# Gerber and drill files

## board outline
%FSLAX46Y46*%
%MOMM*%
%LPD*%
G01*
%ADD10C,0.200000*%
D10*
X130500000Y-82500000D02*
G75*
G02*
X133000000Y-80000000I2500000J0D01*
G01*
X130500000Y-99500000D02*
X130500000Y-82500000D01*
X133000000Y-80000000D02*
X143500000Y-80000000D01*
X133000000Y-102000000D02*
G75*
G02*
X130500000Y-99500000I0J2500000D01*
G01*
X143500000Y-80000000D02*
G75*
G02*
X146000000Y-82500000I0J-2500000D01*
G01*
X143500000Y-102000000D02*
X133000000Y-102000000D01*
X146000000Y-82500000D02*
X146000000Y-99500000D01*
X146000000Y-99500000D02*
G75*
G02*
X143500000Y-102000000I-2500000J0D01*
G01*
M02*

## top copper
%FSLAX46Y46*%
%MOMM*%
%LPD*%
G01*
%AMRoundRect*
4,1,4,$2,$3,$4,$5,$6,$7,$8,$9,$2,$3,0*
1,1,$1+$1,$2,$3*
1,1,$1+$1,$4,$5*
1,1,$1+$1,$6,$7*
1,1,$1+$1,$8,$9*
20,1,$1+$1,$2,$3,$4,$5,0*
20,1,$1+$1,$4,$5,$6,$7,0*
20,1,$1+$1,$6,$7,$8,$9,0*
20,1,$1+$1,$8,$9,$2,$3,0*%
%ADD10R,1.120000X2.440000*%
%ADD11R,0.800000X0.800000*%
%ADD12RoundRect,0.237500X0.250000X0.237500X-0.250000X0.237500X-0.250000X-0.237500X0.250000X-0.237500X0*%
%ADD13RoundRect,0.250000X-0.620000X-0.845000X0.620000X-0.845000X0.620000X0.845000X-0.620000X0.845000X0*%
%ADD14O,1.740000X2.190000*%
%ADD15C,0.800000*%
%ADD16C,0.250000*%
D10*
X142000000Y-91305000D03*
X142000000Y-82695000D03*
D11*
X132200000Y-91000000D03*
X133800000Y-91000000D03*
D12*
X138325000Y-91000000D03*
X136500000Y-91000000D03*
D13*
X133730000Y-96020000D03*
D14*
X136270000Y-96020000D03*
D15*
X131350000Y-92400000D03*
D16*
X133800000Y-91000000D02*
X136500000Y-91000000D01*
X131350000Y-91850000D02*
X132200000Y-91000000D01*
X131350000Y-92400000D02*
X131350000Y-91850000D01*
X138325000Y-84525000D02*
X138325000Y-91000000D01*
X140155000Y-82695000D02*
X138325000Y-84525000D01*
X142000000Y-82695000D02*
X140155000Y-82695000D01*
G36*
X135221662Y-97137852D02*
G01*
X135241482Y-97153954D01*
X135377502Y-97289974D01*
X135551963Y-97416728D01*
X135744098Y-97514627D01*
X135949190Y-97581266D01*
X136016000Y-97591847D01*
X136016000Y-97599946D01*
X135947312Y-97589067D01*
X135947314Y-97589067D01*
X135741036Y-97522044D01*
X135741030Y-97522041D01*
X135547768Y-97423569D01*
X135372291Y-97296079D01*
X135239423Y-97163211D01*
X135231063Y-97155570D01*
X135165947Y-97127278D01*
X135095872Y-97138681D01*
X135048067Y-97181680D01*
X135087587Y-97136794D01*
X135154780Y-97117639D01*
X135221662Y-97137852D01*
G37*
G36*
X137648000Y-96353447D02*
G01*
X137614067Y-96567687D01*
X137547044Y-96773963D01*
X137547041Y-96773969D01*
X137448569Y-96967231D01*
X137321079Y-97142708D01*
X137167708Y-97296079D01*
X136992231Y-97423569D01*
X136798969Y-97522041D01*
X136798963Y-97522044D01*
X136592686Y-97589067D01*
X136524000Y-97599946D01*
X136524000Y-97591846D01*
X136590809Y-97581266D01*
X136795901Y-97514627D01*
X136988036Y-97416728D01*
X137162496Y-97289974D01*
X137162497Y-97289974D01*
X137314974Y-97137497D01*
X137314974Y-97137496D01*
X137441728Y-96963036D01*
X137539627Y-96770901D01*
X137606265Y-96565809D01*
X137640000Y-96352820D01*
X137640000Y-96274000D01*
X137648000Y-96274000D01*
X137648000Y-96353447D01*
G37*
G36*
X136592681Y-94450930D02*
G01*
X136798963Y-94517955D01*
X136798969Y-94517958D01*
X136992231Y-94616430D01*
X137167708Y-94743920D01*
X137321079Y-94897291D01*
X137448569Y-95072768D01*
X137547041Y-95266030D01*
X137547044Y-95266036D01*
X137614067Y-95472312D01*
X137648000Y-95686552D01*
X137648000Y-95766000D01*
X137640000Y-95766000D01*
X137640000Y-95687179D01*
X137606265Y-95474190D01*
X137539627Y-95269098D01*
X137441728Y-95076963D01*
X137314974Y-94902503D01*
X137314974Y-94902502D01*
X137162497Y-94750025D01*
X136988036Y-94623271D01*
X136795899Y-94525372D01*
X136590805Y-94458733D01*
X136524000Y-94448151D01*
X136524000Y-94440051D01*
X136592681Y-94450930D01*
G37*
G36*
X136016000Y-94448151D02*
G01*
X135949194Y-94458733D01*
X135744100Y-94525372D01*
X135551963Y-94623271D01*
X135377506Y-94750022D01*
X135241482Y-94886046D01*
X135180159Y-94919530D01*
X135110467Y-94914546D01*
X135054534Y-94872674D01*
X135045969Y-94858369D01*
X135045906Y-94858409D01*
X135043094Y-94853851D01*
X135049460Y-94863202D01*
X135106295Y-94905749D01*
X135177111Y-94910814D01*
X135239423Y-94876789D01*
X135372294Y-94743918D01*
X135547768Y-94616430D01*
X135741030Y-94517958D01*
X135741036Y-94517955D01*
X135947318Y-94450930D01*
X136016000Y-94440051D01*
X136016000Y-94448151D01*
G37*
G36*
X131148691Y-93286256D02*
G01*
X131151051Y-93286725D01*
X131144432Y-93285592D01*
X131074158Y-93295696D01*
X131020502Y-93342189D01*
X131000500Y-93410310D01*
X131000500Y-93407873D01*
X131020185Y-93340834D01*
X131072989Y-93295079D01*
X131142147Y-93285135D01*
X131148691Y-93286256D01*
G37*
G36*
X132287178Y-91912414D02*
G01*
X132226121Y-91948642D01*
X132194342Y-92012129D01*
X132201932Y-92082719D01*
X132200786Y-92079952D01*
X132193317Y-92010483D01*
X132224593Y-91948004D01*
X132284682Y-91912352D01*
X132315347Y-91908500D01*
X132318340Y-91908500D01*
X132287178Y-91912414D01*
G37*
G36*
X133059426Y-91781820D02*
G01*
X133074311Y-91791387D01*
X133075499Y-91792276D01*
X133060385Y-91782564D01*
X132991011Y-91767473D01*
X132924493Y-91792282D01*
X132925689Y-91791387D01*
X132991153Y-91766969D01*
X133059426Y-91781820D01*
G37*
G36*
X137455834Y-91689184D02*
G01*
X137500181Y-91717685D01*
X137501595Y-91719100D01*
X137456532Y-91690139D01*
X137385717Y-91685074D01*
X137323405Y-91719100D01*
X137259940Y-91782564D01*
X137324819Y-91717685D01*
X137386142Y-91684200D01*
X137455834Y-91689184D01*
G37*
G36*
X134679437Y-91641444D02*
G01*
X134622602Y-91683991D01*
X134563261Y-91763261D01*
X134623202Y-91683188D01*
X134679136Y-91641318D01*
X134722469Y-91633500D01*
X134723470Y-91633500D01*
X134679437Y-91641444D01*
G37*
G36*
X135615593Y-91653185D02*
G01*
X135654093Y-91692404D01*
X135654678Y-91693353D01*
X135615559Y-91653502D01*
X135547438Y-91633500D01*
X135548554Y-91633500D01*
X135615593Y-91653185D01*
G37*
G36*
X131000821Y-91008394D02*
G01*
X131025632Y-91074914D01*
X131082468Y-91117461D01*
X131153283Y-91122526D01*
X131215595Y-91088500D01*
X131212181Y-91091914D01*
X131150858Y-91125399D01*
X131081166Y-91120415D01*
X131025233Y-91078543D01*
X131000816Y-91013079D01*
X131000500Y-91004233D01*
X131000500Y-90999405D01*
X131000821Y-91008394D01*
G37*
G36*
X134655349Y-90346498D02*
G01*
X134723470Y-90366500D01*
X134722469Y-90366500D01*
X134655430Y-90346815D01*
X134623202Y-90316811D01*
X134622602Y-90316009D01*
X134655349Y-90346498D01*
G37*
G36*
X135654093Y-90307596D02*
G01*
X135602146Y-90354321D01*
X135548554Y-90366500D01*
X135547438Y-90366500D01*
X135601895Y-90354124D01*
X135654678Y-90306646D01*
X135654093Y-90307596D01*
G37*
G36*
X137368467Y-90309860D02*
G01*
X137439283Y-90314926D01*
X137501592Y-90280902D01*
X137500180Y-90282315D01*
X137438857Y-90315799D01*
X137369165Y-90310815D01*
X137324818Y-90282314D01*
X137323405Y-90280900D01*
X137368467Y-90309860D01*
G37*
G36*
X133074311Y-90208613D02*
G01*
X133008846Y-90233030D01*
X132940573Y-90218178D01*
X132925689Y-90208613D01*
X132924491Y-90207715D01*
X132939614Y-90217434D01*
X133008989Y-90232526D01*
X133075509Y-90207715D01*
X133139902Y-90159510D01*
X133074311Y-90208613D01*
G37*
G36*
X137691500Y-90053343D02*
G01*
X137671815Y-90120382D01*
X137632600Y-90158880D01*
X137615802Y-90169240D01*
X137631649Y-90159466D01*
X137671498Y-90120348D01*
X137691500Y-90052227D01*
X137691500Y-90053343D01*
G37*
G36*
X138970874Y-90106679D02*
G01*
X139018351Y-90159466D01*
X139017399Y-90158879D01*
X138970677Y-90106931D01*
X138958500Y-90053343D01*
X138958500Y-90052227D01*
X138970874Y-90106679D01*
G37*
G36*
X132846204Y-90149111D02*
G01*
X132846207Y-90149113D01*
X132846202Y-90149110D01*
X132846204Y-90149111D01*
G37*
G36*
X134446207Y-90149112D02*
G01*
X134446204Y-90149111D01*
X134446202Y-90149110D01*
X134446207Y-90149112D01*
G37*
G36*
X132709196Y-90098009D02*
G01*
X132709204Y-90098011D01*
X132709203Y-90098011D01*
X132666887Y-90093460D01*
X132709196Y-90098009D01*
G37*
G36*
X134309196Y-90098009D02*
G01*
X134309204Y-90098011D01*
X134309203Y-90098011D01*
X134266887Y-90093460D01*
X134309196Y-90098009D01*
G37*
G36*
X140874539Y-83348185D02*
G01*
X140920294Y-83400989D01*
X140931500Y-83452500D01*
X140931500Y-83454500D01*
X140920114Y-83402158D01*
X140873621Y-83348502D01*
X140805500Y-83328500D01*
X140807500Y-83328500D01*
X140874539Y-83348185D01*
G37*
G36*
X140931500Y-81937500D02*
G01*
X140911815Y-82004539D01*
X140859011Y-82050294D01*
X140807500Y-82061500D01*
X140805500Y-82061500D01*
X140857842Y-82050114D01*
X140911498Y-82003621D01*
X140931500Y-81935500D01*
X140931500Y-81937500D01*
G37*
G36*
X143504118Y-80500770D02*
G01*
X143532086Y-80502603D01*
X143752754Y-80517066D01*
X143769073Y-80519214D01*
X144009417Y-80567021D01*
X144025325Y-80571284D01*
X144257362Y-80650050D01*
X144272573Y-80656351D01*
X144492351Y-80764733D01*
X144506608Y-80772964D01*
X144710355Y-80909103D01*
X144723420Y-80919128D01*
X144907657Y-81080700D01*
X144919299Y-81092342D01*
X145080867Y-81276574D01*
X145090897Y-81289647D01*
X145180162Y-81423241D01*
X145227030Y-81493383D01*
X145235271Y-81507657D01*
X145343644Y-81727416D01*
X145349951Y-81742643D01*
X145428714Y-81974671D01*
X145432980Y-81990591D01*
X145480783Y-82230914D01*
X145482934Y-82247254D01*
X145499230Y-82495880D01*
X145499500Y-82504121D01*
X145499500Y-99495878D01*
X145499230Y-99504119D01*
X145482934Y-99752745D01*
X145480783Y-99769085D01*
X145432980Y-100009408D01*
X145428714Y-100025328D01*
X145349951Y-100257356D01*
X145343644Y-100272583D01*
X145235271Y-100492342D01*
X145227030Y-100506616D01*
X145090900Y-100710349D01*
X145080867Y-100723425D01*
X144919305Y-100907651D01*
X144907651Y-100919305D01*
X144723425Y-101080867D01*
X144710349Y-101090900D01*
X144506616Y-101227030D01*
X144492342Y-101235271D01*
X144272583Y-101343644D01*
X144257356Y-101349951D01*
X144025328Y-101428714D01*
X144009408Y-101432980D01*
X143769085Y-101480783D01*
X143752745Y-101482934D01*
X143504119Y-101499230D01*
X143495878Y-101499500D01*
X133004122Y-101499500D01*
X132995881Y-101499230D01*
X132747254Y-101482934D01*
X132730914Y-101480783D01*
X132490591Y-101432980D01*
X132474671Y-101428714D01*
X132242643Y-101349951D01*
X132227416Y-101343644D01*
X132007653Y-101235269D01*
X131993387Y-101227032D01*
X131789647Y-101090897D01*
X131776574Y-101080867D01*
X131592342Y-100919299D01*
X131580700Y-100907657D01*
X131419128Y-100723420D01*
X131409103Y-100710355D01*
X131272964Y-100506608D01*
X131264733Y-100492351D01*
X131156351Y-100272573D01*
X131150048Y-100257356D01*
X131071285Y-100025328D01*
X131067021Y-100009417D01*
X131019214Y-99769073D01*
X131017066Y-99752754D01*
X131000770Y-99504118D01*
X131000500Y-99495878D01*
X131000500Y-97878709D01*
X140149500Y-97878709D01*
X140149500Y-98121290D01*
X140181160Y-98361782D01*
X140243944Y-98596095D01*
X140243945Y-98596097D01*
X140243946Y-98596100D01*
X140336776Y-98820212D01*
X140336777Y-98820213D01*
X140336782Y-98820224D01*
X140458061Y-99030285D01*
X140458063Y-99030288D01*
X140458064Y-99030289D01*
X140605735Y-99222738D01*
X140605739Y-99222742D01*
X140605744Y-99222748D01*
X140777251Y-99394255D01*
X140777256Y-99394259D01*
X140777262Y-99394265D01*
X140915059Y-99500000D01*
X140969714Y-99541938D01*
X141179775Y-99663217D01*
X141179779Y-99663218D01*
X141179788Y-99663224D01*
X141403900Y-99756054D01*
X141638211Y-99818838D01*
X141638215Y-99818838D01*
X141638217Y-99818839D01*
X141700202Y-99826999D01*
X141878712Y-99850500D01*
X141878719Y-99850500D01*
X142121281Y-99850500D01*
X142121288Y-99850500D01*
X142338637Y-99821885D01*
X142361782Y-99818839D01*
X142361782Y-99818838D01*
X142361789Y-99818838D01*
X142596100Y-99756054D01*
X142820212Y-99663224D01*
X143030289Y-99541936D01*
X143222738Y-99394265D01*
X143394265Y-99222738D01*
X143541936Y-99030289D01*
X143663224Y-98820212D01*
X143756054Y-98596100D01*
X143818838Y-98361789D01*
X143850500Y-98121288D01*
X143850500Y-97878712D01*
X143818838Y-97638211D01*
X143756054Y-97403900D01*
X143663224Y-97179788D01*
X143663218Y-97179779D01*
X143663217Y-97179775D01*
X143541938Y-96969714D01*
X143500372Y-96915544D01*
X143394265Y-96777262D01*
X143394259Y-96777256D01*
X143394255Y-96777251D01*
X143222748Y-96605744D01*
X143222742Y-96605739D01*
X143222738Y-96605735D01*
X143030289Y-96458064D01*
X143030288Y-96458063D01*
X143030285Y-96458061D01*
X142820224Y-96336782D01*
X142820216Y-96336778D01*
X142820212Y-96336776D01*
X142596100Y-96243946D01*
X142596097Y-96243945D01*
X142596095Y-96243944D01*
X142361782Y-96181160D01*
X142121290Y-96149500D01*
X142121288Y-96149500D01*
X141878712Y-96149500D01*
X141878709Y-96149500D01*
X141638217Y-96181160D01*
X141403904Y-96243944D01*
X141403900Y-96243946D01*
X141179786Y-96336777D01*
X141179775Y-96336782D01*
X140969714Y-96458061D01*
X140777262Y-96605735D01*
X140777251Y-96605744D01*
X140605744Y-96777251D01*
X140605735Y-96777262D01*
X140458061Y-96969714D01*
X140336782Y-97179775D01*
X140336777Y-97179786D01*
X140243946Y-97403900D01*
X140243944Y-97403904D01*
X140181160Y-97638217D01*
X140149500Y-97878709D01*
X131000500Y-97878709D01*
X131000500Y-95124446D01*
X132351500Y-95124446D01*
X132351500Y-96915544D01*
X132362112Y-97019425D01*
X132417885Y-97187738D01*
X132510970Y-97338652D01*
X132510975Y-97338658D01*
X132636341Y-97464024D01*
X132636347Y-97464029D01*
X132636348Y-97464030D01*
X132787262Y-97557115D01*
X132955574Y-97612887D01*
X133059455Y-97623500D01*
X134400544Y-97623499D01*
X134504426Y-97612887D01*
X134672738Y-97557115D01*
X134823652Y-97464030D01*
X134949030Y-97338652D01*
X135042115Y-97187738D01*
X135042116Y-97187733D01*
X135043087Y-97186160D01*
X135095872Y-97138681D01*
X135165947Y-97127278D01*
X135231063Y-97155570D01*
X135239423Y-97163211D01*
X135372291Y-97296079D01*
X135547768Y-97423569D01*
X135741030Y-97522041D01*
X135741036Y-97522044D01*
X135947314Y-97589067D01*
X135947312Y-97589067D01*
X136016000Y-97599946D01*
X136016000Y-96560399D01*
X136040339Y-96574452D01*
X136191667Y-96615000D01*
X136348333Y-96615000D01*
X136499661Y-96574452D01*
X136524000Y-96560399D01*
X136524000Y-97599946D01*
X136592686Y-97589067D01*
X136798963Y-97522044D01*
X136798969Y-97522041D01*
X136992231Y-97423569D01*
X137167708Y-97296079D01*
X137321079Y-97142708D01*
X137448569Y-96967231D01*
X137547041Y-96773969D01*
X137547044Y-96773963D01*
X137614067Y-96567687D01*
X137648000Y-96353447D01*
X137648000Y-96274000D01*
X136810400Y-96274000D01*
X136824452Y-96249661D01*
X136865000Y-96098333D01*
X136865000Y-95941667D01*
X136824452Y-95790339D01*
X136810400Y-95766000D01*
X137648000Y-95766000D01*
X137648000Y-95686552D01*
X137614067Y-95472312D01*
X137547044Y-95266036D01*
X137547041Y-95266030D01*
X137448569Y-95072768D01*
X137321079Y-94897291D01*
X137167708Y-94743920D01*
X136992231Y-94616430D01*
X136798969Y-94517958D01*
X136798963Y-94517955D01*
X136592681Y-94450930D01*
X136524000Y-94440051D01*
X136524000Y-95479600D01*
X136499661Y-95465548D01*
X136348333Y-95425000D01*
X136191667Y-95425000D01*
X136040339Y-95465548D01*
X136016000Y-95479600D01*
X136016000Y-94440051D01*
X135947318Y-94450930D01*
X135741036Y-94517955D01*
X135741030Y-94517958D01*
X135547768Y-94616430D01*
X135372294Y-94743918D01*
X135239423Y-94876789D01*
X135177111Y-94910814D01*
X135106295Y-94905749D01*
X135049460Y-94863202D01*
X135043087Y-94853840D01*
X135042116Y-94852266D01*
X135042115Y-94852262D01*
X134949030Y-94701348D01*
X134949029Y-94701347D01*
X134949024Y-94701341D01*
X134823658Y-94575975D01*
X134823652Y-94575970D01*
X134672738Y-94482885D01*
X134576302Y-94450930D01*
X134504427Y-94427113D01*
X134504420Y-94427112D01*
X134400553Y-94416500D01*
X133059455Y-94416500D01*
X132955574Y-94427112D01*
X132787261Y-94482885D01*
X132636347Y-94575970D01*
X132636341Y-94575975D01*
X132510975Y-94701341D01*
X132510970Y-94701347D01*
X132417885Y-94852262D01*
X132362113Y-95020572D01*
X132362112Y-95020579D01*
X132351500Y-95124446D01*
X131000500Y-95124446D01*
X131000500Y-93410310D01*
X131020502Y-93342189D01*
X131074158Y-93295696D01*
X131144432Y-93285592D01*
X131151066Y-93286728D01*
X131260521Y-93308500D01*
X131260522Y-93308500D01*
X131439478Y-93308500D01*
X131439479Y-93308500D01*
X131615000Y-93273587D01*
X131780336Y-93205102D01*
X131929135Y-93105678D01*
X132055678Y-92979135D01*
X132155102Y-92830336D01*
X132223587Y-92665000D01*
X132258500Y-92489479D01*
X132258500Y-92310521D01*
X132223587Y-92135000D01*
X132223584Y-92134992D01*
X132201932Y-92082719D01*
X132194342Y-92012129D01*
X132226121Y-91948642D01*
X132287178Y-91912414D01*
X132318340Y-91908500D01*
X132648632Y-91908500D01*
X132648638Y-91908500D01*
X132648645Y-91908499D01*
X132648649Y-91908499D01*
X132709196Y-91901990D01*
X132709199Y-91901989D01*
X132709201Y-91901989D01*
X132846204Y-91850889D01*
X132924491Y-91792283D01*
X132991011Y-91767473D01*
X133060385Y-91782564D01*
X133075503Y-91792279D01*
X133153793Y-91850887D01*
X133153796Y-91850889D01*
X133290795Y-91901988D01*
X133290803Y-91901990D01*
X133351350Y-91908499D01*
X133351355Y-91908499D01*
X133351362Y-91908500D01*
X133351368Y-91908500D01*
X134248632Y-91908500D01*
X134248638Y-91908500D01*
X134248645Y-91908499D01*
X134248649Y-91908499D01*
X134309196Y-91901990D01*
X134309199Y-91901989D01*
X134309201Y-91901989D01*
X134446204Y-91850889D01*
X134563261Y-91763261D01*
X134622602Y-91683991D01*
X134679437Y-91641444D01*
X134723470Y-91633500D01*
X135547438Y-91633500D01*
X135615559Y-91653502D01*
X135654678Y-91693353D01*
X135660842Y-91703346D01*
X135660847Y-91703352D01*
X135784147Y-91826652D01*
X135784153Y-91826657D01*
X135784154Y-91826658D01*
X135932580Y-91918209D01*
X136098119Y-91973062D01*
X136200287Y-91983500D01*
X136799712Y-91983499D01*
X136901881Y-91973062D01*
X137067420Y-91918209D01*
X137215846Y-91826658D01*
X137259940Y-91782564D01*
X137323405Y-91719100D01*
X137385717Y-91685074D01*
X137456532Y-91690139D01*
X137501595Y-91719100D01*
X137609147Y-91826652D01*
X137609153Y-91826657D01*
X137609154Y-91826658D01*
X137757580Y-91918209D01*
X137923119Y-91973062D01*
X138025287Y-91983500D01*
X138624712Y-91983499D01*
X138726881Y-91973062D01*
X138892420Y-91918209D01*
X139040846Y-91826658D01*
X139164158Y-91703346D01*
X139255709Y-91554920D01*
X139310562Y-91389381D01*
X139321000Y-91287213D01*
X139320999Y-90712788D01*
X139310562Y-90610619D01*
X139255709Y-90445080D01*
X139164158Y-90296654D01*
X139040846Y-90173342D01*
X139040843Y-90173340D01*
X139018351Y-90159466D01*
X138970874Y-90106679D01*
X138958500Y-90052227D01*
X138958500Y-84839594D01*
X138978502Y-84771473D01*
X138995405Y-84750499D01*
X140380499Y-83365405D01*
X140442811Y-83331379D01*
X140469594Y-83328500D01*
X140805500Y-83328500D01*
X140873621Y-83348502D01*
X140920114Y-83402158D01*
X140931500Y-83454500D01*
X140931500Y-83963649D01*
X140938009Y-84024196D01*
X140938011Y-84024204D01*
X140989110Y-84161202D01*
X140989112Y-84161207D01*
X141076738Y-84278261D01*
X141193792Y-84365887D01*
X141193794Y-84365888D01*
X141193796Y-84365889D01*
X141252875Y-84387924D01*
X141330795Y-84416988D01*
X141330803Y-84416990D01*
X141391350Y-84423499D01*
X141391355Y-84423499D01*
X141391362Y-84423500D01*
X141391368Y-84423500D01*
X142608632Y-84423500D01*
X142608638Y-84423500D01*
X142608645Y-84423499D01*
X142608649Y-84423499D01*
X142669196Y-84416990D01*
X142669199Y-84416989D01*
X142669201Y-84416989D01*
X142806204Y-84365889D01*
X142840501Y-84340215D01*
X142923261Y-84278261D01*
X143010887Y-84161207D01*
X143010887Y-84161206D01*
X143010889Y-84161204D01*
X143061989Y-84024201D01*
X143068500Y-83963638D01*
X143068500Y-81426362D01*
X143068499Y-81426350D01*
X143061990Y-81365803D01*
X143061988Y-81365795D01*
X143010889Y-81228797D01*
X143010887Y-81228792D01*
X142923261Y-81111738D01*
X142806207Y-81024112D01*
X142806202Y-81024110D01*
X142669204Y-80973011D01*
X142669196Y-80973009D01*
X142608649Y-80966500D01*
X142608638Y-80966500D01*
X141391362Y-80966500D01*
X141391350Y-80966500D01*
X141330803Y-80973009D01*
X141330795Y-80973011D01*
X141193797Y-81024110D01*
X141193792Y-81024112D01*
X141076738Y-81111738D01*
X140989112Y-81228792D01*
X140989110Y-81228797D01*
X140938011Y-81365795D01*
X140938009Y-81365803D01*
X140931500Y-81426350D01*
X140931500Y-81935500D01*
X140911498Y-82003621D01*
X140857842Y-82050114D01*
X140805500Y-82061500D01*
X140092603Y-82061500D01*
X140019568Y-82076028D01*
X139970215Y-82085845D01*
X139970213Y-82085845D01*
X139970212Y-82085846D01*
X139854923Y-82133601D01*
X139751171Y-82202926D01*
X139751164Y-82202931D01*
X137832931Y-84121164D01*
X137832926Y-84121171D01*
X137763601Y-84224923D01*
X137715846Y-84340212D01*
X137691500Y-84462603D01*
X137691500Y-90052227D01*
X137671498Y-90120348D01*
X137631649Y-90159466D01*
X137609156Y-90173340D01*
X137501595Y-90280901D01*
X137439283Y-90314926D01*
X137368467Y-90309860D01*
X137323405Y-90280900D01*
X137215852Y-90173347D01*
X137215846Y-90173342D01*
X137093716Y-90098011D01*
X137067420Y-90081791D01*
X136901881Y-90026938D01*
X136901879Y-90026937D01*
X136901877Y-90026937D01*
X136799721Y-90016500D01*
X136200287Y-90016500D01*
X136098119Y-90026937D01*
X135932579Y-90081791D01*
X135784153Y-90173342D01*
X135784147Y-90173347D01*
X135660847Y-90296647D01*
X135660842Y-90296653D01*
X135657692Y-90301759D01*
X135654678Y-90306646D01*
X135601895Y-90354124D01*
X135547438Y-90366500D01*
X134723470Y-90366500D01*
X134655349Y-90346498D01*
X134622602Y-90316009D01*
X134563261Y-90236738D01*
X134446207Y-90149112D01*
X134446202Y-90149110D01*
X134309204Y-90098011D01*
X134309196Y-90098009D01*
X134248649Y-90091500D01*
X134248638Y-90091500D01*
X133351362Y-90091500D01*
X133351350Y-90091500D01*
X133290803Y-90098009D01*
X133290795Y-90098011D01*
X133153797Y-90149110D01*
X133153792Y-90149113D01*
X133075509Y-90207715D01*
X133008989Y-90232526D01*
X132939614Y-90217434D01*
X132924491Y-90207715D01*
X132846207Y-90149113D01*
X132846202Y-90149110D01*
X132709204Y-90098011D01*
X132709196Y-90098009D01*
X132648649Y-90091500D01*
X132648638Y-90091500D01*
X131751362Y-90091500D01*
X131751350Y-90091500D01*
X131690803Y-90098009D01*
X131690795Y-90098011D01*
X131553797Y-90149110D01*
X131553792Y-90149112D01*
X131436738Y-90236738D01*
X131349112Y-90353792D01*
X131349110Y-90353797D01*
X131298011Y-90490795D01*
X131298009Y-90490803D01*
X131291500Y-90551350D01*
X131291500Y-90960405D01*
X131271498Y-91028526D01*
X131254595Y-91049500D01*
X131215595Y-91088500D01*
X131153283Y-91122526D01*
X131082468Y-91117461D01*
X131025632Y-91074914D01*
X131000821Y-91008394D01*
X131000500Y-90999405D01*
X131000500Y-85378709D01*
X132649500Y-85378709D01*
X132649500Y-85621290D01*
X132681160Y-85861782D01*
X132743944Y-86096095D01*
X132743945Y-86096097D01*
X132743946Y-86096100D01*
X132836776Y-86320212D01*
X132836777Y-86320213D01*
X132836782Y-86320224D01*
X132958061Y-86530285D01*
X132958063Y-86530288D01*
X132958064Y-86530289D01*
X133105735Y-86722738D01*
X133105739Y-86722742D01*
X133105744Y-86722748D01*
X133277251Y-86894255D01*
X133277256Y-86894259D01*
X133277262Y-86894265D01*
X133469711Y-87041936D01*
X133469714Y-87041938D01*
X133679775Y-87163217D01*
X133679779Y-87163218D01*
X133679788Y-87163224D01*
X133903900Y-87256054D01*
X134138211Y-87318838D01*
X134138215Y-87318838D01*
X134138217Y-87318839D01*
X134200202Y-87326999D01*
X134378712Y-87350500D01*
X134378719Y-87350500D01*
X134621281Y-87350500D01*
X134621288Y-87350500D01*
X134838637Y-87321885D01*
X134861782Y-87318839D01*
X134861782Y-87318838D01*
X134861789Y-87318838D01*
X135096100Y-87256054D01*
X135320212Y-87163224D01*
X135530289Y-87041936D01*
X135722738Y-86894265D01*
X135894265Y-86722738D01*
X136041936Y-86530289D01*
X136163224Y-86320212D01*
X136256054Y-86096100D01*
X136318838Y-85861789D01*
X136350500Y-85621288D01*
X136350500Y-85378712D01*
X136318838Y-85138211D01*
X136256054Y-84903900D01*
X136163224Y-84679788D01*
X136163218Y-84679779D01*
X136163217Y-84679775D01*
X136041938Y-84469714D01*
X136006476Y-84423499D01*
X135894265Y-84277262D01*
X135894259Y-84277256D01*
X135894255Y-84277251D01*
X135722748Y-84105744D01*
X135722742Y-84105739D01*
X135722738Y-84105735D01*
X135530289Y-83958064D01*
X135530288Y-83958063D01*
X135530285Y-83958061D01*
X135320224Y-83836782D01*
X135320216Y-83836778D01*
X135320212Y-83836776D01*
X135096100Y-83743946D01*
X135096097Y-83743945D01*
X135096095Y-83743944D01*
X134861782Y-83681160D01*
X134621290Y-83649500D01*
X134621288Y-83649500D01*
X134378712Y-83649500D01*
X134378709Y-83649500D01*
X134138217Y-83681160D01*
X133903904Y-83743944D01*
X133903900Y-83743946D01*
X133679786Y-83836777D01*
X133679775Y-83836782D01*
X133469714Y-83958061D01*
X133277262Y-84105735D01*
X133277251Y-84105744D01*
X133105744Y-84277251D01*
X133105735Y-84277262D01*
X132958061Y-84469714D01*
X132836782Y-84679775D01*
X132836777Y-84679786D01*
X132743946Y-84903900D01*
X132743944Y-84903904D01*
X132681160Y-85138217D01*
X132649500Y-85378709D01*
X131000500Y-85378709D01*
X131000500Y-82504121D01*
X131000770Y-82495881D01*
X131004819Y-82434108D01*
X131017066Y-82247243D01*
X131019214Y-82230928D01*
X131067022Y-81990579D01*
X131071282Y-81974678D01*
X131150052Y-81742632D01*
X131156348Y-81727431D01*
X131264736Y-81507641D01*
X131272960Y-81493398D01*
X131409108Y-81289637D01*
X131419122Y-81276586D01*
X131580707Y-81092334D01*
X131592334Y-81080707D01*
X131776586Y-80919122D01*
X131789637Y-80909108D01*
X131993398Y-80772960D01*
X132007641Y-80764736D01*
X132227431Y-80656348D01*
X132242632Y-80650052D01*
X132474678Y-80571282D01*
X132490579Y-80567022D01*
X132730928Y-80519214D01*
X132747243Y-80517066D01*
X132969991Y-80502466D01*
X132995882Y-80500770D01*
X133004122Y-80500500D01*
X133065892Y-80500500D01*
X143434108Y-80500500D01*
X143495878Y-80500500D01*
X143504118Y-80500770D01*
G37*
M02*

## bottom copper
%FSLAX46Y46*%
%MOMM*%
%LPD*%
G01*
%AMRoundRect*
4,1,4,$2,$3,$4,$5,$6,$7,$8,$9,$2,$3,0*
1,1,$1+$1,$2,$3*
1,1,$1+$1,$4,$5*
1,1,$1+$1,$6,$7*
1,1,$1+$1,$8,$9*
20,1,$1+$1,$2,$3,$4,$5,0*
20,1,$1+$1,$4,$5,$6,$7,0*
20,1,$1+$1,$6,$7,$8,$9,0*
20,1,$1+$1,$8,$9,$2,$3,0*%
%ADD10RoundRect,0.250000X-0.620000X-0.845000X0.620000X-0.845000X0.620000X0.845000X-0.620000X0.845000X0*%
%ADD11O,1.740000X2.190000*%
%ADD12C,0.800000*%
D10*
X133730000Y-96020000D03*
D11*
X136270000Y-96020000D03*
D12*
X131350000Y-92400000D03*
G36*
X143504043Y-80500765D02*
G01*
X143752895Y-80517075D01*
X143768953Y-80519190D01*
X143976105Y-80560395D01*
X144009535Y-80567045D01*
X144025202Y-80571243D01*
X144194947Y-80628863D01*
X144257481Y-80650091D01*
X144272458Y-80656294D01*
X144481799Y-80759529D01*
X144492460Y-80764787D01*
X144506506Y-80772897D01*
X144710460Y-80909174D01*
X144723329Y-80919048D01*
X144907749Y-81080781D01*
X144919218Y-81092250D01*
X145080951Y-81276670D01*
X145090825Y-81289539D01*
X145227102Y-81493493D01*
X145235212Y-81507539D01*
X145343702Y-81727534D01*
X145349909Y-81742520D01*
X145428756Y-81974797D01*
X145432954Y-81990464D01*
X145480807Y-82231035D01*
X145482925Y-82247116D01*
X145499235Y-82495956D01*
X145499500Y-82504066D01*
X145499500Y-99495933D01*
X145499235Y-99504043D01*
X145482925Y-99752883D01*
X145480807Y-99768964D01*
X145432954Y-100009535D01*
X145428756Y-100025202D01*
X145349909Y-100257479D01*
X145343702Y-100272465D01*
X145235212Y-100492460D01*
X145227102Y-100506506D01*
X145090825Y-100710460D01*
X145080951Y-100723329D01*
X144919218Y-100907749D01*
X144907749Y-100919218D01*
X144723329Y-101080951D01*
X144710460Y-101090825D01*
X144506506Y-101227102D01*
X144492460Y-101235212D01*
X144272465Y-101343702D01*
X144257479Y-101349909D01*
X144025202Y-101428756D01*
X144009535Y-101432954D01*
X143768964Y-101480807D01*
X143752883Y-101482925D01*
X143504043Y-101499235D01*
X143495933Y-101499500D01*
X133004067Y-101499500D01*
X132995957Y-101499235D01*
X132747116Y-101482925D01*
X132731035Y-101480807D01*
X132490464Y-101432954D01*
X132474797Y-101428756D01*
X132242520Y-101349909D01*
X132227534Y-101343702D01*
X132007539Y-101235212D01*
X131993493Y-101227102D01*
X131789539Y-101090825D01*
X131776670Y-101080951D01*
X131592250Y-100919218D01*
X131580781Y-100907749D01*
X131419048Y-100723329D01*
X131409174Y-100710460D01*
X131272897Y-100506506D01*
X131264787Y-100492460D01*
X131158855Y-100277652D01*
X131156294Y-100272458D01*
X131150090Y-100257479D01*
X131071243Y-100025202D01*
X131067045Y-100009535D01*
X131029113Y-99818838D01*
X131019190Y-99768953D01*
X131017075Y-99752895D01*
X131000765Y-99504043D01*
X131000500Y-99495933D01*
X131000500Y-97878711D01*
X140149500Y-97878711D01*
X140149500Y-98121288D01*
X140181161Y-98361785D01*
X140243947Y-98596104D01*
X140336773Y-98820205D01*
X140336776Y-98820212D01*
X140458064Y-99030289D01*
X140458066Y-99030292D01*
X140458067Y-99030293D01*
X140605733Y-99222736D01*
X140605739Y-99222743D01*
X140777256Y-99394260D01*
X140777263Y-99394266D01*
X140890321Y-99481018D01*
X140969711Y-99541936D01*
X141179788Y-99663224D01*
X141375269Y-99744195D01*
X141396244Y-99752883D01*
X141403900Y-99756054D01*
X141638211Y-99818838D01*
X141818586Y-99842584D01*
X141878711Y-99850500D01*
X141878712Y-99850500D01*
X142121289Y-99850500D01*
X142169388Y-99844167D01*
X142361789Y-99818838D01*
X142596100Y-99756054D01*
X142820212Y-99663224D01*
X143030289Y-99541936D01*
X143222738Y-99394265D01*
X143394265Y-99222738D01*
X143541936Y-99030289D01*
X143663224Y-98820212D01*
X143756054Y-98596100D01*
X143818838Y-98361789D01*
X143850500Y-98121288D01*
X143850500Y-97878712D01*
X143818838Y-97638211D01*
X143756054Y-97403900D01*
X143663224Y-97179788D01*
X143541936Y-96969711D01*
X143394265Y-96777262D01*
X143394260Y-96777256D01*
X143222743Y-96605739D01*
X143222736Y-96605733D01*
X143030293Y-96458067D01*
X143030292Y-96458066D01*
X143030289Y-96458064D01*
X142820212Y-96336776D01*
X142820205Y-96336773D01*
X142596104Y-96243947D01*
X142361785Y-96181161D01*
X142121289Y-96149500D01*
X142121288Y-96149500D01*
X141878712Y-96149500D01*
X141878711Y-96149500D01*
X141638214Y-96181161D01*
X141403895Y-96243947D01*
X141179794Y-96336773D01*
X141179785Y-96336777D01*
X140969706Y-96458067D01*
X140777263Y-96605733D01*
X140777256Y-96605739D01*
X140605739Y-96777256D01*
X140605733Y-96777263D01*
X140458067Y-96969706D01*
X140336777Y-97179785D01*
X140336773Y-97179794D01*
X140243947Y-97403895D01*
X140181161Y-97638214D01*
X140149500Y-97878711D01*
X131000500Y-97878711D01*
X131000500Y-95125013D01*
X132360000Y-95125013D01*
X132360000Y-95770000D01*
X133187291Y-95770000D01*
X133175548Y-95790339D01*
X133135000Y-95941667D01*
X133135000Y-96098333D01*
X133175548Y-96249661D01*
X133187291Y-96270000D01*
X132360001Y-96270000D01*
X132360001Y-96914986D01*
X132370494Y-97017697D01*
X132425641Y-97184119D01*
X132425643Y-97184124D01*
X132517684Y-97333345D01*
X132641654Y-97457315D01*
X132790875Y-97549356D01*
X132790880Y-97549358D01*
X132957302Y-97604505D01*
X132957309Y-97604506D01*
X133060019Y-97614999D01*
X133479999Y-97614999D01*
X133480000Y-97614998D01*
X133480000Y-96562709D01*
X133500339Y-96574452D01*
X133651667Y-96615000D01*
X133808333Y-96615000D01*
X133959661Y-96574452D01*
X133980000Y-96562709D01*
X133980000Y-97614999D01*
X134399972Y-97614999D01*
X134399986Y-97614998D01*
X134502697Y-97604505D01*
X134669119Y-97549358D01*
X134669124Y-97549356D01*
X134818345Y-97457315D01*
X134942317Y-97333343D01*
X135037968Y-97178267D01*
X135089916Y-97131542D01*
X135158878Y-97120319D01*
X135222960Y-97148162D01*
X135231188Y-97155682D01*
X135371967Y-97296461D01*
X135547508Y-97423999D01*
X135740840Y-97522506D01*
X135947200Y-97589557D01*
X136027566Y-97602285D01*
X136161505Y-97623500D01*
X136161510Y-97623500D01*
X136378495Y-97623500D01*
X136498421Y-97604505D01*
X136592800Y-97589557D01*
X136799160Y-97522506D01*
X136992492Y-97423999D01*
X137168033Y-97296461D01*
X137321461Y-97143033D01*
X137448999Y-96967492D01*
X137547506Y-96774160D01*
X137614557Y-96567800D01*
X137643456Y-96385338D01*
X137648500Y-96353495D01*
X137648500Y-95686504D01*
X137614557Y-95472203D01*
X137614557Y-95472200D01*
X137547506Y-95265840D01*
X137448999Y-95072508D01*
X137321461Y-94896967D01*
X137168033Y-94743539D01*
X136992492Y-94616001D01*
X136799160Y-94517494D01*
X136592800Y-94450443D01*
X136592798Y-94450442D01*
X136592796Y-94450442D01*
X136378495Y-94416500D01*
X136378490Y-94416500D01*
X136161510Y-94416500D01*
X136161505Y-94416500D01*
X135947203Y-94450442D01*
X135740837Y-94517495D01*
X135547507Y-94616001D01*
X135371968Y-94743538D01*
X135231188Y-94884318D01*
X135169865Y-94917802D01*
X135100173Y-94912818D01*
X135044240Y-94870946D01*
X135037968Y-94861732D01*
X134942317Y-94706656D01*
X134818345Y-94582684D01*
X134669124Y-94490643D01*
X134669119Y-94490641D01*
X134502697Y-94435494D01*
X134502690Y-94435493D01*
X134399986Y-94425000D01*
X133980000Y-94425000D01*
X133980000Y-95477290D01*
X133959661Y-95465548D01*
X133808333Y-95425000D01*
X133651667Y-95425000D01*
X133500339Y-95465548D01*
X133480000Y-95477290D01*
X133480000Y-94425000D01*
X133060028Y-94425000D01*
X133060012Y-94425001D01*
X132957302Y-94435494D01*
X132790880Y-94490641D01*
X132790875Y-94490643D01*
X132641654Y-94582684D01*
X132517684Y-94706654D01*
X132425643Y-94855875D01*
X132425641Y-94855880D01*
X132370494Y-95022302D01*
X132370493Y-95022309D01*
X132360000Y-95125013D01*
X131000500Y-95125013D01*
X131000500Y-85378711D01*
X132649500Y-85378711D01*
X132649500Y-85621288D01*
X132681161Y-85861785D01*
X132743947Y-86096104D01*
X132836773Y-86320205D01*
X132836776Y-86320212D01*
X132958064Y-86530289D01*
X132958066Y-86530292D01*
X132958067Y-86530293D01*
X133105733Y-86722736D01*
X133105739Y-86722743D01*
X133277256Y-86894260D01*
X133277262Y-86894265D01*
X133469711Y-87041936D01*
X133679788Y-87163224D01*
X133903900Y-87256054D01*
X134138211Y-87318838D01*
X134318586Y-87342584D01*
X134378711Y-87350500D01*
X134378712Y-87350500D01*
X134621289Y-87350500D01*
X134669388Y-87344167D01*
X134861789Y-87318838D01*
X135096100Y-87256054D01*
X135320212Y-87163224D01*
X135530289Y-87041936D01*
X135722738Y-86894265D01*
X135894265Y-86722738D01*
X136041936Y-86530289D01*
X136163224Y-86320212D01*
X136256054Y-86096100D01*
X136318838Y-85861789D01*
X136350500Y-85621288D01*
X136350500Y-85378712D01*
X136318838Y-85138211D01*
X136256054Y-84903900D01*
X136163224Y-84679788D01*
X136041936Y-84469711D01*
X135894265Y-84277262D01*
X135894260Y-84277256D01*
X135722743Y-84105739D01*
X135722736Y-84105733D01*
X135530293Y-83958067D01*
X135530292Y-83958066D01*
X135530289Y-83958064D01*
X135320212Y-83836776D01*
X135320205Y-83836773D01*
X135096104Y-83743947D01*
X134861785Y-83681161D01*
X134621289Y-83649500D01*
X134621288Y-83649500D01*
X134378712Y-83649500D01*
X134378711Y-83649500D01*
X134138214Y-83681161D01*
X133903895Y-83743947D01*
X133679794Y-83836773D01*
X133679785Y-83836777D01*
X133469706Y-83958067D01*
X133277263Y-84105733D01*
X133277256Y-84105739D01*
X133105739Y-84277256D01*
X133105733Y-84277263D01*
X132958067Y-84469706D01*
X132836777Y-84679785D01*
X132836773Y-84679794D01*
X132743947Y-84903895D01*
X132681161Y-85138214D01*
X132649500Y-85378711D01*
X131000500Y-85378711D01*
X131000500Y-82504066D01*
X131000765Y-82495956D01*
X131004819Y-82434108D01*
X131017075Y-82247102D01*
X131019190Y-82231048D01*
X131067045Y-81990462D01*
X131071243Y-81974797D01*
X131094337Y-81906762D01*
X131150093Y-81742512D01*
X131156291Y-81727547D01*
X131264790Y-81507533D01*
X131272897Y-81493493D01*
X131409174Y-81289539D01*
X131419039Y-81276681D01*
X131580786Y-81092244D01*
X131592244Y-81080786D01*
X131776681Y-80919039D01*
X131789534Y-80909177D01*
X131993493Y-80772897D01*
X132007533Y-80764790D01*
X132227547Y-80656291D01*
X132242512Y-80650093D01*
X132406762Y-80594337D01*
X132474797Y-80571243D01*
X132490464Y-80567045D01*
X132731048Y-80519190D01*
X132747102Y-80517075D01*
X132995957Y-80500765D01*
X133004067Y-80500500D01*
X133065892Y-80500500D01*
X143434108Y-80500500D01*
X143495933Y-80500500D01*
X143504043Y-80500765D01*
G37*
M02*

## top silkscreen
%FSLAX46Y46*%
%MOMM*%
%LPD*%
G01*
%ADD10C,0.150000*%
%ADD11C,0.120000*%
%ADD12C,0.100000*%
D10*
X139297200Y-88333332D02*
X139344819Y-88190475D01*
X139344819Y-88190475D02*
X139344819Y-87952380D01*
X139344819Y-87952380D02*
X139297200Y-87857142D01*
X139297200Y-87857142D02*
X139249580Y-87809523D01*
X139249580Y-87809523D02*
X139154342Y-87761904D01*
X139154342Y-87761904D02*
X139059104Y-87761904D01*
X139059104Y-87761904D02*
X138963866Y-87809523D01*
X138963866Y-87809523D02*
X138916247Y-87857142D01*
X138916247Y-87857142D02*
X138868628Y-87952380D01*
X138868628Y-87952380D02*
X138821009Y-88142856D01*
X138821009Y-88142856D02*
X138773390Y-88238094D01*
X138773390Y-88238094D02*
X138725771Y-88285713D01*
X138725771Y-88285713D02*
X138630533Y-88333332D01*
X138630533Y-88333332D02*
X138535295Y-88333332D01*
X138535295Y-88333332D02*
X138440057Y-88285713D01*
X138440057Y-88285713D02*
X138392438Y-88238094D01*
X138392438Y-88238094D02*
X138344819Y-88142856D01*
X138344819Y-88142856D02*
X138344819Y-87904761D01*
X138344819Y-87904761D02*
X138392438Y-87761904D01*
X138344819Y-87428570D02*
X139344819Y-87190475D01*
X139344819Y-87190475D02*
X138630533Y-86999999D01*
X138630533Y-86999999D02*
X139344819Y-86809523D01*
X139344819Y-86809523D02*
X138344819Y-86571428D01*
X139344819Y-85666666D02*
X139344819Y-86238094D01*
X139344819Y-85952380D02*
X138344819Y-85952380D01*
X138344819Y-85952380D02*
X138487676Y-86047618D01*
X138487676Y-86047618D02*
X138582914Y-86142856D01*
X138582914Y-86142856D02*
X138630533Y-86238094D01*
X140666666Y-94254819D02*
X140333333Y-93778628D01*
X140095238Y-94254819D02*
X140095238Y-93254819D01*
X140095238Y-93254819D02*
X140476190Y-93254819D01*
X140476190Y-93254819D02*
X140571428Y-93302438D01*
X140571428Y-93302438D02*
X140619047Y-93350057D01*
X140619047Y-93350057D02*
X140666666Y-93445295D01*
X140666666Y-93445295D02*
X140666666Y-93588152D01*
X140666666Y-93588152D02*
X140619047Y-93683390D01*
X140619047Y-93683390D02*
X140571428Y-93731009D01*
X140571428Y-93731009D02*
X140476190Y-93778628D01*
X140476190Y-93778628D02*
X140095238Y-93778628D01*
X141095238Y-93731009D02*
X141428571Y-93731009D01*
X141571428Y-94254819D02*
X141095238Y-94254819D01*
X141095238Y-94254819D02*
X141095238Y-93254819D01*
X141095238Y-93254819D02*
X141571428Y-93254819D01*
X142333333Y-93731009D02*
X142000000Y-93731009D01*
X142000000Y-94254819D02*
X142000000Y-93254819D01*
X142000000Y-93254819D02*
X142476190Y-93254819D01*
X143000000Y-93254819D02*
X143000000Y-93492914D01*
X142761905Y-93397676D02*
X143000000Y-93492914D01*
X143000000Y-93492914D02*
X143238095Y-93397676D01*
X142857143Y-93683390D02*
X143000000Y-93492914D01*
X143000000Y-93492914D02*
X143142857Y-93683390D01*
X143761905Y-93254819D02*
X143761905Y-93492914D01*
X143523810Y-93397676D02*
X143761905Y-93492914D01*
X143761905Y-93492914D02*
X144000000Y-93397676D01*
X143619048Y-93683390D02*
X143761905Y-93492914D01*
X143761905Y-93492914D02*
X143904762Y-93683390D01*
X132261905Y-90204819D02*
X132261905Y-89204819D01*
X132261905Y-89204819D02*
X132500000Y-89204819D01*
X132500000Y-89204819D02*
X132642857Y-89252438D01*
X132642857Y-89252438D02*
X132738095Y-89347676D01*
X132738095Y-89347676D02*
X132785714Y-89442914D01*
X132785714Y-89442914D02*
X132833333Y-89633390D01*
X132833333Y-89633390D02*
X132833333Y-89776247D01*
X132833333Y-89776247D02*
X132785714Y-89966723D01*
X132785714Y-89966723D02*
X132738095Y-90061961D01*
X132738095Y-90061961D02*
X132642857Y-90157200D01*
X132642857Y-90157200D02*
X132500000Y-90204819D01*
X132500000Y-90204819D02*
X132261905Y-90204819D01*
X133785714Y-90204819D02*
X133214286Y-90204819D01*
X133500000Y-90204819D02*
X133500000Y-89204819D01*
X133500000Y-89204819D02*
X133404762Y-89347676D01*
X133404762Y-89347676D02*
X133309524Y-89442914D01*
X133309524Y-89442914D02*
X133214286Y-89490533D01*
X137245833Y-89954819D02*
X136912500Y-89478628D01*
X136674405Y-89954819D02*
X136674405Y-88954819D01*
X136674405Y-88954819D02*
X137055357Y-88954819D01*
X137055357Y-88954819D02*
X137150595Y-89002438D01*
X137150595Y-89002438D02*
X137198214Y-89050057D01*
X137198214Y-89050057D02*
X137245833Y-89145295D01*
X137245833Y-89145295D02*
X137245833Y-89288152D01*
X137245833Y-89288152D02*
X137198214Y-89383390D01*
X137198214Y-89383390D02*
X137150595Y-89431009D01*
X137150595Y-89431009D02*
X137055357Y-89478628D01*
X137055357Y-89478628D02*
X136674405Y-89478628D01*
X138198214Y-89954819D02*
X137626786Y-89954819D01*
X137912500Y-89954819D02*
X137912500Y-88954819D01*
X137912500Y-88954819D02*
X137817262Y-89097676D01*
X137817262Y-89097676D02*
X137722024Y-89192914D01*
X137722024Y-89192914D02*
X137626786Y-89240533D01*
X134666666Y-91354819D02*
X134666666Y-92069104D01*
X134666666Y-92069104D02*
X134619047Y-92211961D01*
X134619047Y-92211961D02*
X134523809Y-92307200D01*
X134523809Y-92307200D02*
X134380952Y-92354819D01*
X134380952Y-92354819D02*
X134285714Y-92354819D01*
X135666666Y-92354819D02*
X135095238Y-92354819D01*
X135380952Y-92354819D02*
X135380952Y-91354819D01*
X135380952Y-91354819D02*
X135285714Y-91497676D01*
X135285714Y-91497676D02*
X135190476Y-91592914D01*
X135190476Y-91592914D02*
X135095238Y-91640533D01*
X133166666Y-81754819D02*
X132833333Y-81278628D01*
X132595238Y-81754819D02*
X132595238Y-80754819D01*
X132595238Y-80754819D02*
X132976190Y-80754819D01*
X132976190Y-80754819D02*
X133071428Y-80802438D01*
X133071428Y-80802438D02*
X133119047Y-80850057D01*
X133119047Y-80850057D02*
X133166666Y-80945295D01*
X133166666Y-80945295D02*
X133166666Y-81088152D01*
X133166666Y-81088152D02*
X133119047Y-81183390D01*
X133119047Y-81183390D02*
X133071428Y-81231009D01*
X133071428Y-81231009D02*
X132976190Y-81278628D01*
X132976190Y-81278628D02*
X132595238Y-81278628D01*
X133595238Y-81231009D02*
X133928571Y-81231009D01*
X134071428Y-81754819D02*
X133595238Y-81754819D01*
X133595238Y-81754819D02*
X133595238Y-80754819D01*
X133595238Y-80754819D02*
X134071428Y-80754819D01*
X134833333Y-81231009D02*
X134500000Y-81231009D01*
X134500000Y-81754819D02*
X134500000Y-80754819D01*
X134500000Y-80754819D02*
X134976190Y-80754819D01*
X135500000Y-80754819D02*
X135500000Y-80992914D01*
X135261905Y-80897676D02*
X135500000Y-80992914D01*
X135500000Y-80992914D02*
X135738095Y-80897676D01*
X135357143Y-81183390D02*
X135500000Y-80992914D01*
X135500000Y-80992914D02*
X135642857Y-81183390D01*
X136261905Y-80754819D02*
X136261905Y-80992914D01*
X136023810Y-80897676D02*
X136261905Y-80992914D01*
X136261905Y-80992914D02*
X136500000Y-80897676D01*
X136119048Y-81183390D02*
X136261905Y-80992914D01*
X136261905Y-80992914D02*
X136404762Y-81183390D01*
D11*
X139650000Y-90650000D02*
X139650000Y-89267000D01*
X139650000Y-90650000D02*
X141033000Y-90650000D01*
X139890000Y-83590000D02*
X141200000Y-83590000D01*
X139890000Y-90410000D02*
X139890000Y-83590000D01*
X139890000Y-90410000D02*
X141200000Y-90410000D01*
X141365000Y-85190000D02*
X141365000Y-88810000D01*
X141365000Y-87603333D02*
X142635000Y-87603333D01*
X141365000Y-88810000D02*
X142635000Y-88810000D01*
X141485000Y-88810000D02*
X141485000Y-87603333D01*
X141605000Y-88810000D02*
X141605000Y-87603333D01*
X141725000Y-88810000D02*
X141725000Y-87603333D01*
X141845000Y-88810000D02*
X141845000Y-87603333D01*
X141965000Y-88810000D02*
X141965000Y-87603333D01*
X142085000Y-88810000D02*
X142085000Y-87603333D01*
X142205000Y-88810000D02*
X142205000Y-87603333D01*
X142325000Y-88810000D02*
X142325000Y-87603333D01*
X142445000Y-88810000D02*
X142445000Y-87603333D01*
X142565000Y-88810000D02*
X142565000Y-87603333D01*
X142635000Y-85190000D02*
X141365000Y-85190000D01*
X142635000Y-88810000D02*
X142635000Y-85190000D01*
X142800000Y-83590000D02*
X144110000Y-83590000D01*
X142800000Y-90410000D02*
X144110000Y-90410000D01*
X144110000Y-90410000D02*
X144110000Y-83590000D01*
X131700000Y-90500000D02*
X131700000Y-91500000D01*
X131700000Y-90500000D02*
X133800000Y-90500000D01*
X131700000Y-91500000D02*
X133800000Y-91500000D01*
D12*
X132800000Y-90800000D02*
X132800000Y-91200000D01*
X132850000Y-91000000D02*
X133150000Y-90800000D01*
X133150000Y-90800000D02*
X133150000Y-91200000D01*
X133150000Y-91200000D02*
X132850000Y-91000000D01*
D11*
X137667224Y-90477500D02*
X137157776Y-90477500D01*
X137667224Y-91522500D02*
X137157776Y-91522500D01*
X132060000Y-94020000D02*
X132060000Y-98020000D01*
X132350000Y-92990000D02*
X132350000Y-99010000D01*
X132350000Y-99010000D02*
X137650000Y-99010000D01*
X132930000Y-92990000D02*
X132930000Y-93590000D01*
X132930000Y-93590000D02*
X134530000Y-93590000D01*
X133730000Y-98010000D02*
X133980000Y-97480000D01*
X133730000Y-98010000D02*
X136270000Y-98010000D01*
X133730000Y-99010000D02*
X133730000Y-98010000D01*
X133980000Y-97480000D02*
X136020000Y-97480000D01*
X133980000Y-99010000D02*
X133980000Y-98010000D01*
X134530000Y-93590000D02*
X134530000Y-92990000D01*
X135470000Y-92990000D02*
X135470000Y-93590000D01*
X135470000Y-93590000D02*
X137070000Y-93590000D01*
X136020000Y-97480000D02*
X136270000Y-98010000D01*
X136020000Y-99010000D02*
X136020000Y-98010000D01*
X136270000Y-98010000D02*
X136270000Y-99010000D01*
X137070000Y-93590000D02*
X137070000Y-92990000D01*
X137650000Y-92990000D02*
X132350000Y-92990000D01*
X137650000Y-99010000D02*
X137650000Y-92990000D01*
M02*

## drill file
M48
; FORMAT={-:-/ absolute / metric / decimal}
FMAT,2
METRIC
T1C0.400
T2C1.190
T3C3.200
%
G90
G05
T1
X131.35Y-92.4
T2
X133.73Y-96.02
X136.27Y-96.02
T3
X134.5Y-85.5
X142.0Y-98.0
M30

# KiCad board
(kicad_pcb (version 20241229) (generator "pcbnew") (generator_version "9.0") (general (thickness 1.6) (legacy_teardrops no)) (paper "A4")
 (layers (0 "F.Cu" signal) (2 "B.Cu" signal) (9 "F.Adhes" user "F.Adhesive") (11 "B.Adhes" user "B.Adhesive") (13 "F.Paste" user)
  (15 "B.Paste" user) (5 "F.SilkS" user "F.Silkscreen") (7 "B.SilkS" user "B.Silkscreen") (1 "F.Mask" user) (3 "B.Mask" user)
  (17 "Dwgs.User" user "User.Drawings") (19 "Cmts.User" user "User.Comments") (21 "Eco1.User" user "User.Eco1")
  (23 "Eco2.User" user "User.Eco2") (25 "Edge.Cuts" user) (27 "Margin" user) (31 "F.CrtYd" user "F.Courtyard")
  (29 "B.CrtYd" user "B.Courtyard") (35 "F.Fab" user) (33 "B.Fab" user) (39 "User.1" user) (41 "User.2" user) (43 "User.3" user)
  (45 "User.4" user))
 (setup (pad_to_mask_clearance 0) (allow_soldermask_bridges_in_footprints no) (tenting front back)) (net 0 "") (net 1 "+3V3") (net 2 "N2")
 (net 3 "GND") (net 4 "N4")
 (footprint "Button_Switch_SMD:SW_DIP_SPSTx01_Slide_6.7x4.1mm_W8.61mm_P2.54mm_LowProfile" (layer "F.Cu") (at 142 87 90)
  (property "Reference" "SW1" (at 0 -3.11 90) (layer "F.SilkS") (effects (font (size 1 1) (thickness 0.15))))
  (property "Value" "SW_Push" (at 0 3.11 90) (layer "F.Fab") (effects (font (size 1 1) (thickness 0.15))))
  (fp_line (start -3.65 -2.35) (end -2.267 -2.35) (stroke (width 0.12) (type solid)) (layer "F.SilkS"))
  (fp_line (start -3.65 -2.35) (end -3.65 -0.967) (stroke (width 0.12) (type solid)) (layer "F.SilkS"))
  (fp_line (start 3.41 -2.11) (end 3.41 -0.8) (stroke (width 0.12) (type solid)) (layer "F.SilkS"))
  (fp_line (start -3.41 -2.11) (end 3.41 -2.11) (stroke (width 0.12) (type solid)) (layer "F.SilkS"))
  (fp_line (start -3.41 -2.11) (end -3.41 -0.8) (stroke (width 0.12) (type solid)) (layer "F.SilkS"))
  (fp_line (start 1.81 -0.635) (end -1.81 -0.635) (stroke (width 0.12) (type solid)) (layer "F.SilkS"))
  (fp_line (start -0.603333 -0.635) (end -0.603333 0.635) (stroke (width 0.12) (type solid)) (layer "F.SilkS"))
  (fp_line (start -1.81 -0.635) (end -1.81 0.635) (stroke (width 0.12) (type solid)) (layer "F.SilkS"))
  (fp_line (start -1.81 -0.515) (end -0.603333 -0.515) (stroke (width 0.12) (type solid)) (layer "F.SilkS"))
  (fp_line (start -1.81 -0.395) (end -0.603333 -0.395) (stroke (width 0.12) (type solid)) (layer "F.SilkS"))
  (fp_line (start -1.81 -0.275) (end -0.603333 -0.275) (stroke (width 0.12) (type solid)) (layer "F.SilkS"))
  (fp_line (start -1.81 -0.155) (end -0.603333 -0.155) (stroke (width 0.12) (type solid)) (layer "F.SilkS"))
  (fp_line (start -1.81 -0.035) (end -0.603333 -0.035) (stroke (width 0.12) (type solid)) (layer "F.SilkS"))
  (fp_line (start -1.81 0.085) (end -0.603333 0.085) (stroke (width 0.12) (type solid)) (layer "F.SilkS"))
  (fp_line (start -1.81 0.205) (end -0.603333 0.205) (stroke (width 0.12) (type solid)) (layer "F.SilkS"))
  (fp_line (start -1.81 0.325) (end -0.603333 0.325) (stroke (width 0.12) (type solid)) (layer "F.SilkS"))
  (fp_line (start -1.81 0.445) (end -0.603333 0.445) (stroke (width 0.12) (type solid)) (layer "F.SilkS"))
  (fp_line (start -1.81 0.565) (end -0.603333 0.565) (stroke (width 0.12) (type solid)) (layer "F.SilkS"))
  (fp_line (start 1.81 0.635) (end 1.81 -0.635) (stroke (width 0.12) (type solid)) (layer "F.SilkS"))
  (fp_line (start -1.81 0.635) (end 1.81 0.635) (stroke (width 0.12) (type solid)) (layer "F.SilkS"))
  (fp_line (start 3.41 0.8) (end 3.41 2.11) (stroke (width 0.12) (type solid)) (layer "F.SilkS"))
  (fp_line (start -3.41 0.8) (end -3.41 2.11) (stroke (width 0.12) (type solid)) (layer "F.SilkS"))
  (fp_line (start -3.41 2.11) (end 3.41 2.11) (stroke (width 0.12) (type solid)) (layer "F.SilkS"))
  (pad "1" smd rect (at -4.305 0 90) (size 2.44 1.12) (layers "F.Cu" "F.Mask" "F.Paste") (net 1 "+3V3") (zone_connect 2))
  (pad "2" smd rect (at 4.305 0 90) (size 2.44 1.12) (layers "F.Cu" "F.Mask" "F.Paste") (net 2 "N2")))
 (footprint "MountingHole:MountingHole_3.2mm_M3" (layer "F.Cu") (at 142 98)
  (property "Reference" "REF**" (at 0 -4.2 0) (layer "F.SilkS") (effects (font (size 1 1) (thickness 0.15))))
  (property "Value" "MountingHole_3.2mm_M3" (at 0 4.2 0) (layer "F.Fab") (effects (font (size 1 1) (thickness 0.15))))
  (pad "" np_thru_hole circle (at 0 0) (size 3.2 3.2) (drill 3.2) (layers "*.Cu" "*.Mask")))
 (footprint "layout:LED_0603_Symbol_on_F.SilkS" (layer "F.Cu") (at 133 91)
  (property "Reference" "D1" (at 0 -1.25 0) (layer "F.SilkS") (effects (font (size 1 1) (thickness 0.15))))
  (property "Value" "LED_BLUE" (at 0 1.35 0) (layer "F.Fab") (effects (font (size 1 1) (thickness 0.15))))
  (fp_line (start -1.3 -0.5) (end -1.3 0.5) (stroke (width 0.12) (type solid)) (layer "F.SilkS"))
  (fp_line (start -1.3 -0.5) (end 0.8 -0.5) (stroke (width 0.12) (type solid)) (layer "F.SilkS"))
  (fp_line (start -1.3 0.5) (end 0.8 0.5) (stroke (width 0.12) (type solid)) (layer "F.SilkS"))
  (fp_line (start -0.2 -0.2) (end -0.2 0.2) (stroke (width 0.1) (type solid)) (layer "F.SilkS"))
  (fp_line (start -0.15 0) (end 0.15 -0.2) (stroke (width 0.1) (type solid)) (layer "F.SilkS"))
  (fp_line (start 0.15 -0.2) (end 0.15 0.2) (stroke (width 0.1) (type solid)) (layer "F.SilkS"))
  (fp_line (start 0.15 0.2) (end -0.15 0) (stroke (width 0.1) (type solid)) (layer "F.SilkS"))
  (pad "1" smd rect (at -0.8 0 180) (size 0.8 0.8) (layers "F.Cu" "F.Mask" "F.Paste") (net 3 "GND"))
  (pad "2" smd rect (at 0.8 0 180) (size 0.8 0.8) (layers "F.Cu" "F.Mask" "F.Paste") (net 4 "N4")))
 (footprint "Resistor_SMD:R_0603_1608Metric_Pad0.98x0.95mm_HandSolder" (layer "F.Cu") (at 137.4125 91 180)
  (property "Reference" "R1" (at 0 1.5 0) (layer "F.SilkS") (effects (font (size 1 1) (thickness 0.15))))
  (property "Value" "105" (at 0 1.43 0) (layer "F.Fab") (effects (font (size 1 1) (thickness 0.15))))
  (fp_line (start -0.254724 0.5225) (end 0.254724 0.5225) (stroke (width 0.12) (type solid)) (layer "F.SilkS"))
  (fp_line (start -0.254724 -0.5225) (end 0.254724 -0.5225) (stroke (width 0.12) (type solid)) (layer "F.SilkS"))
  (pad "1" smd roundrect (at -0.9125 0 180) (size 0.975 0.95) (layers "F.Cu" "F.Mask" "F.Paste") (roundrect_rratio 0.25) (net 2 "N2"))
  (pad "2" smd roundrect (at 0.9125 0 180) (size 0.975 0.95) (layers "F.Cu" "F.Mask" "F.Paste") (roundrect_rratio 0.25) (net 4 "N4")))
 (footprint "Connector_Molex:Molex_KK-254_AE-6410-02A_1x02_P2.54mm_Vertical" (layer "F.Cu") (at 133.73 96.02)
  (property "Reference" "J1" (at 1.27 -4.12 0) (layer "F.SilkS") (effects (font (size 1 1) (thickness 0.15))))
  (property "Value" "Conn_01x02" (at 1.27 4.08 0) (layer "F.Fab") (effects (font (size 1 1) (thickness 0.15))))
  (fp_line (start -1.67 -2) (end -1.67 2) (stroke (width 0.12) (type solid)) (layer "F.SilkS"))
  (fp_line (start -1.38 -3.03) (end -1.38 2.99) (stroke (width 0.12) (type solid)) (layer "F.SilkS"))
  (fp_line (start -1.38 2.99) (end 3.92 2.99) (stroke (width 0.12) (type solid)) (layer "F.SilkS"))
  (fp_line (start -0.8 -3.03) (end -0.8 -2.43) (stroke (width 0.12) (type solid)) (layer "F.SilkS"))
  (fp_line (start -0.8 -2.43) (end 0.8 -2.43) (stroke (width 0.12) (type solid)) (layer "F.SilkS"))
  (fp_line (start 0 1.99) (end 0.25 1.46) (stroke (width 0.12) (type solid)) (layer "F.SilkS"))
  (fp_line (start 0 1.99) (end 2.54 1.99) (stroke (width 0.12) (type solid)) (layer "F.SilkS"))
  (fp_line (start 0 2.99) (end 0 1.99) (stroke (width 0.12) (type solid)) (layer "F.SilkS"))
  (fp_line (start 0.25 1.46) (end 2.29 1.46) (stroke (width 0.12) (type solid)) (layer "F.SilkS"))
  (fp_line (start 0.25 2.99) (end 0.25 1.99) (stroke (width 0.12) (type solid)) (layer "F.SilkS"))
  (fp_line (start 0.8 -2.43) (end 0.8 -3.03) (stroke (width 0.12) (type solid)) (layer "F.SilkS"))
  (fp_line (start 1.74 -3.03) (end 1.74 -2.43) (stroke (width 0.12) (type solid)) (layer "F.SilkS"))
  (fp_line (start 1.74 -2.43) (end 3.34 -2.43) (stroke (width 0.12) (type solid)) (layer "F.SilkS"))
  (fp_line (start 2.29 1.46) (end 2.54 1.99) (stroke (width 0.12) (type solid)) (layer "F.SilkS"))
  (fp_line (start 2.29 2.99) (end 2.29 1.99) (stroke (width 0.12) (type solid)) (layer "F.SilkS"))
  (fp_line (start 2.54 1.99) (end 2.54 2.99) (stroke (width 0.12) (type solid)) (layer "F.SilkS"))
  (fp_line (start 3.34 -2.43) (end 3.34 -3.03) (stroke (width 0.12) (type solid)) (layer "F.SilkS"))
  (fp_line (start 3.92 -3.03) (end -1.38 -3.03) (stroke (width 0.12) (type solid)) (layer "F.SilkS"))
  (fp_line (start 3.92 2.99) (end 3.92 -3.03) (stroke (width 0.12) (type solid)) (layer "F.SilkS"))
  (pad "1" thru_hole roundrect (at 0 0) (size 1.74 2.19) (drill 1.19) (layers "*.Cu" "*.Mask") (remove_unused_layers no)
   (roundrect_rratio 0.143678) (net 3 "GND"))
  (pad "2" thru_hole oval (at 2.54 0) (size 1.74 2.19) (drill 1.19) (layers "*.Cu" "*.Mask") (remove_unused_layers no) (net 1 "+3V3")))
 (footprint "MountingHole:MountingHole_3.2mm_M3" (layer "F.Cu") (at 134.5 85.5)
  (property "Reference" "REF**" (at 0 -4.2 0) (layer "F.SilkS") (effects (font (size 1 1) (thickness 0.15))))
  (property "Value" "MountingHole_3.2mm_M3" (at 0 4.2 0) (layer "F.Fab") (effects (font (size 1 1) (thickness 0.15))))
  (pad "" np_thru_hole circle (at 0 0) (size 3.2 3.2) (drill 3.2) (layers "*.Cu" "*.Mask")))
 (gr_arc (start 130.5 82.5) (mid 131.232233 80.732233) (end 133 80) (stroke (width 0.2) (type solid)) (layer "Edge.Cuts"))
 (gr_line (start 130.5 99.5) (end 130.5 82.5) (stroke (width 0.2) (type solid)) (layer "Edge.Cuts"))
 (gr_line (start 133 80) (end 143.5 80) (stroke (width 0.2) (type solid)) (layer "Edge.Cuts"))
 (gr_arc (start 133 102) (mid 131.232233 101.267767) (end 130.5 99.5) (stroke (width 0.2) (type solid)) (layer "Edge.Cuts"))
 (gr_arc (start 143.5 80) (mid 145.267767 80.732233) (end 146 82.5) (stroke (width 0.2) (type solid)) (layer "Edge.Cuts"))
 (gr_line (start 143.5 102) (end 133 102) (stroke (width 0.2) (type solid)) (layer "Edge.Cuts"))
 (gr_line (start 146 82.5) (end 146 99.5) (stroke (width 0.2) (type solid)) (layer "Edge.Cuts"))
 (gr_arc (start 146 99.5) (mid 145.267767 101.267767) (end 143.5 102) (stroke (width 0.2) (type solid)) (layer "Edge.Cuts"))
 (segment (start 133.8 91) (end 136.5 91) (width 0.25) (layer "F.Cu") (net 4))
 (segment (start 131.35 91.85) (end 132.2 91) (width 0.25) (layer "F.Cu") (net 3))
 (segment (start 131.35 92.4) (end 131.35 91.85) (width 0.25) (layer "F.Cu") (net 3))
 (via (at 131.35 92.4) (size 0.8) (drill 0.4) (layers "F.Cu" "B.Cu") (free yes) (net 3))
 (segment (start 138.325 84.525) (end 138.325 91) (width 0.25) (layer "F.Cu") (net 2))
 (segment (start 140.155 82.695) (end 138.325 84.525) (width 0.25) (layer "F.Cu") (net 2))
 (segment (start 142 82.695) (end 140.155 82.695) (width 0.25) (layer "F.Cu") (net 2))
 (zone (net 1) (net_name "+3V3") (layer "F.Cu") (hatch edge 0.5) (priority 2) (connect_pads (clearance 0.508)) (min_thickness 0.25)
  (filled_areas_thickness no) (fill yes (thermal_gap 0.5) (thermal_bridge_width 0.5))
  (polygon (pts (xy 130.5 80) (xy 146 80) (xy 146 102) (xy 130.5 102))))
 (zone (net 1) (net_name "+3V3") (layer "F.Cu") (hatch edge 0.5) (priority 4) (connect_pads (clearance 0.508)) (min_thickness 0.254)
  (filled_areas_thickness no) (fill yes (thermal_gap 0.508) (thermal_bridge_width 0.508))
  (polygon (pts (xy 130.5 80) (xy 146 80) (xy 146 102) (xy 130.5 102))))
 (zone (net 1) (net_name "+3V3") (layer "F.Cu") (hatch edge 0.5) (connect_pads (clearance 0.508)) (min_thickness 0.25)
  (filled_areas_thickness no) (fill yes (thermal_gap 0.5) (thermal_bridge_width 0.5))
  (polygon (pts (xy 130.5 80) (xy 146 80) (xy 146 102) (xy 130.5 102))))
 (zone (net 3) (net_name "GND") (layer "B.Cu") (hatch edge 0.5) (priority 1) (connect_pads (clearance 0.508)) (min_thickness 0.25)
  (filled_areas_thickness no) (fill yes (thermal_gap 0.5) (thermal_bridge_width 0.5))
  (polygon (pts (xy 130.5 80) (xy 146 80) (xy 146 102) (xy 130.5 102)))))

